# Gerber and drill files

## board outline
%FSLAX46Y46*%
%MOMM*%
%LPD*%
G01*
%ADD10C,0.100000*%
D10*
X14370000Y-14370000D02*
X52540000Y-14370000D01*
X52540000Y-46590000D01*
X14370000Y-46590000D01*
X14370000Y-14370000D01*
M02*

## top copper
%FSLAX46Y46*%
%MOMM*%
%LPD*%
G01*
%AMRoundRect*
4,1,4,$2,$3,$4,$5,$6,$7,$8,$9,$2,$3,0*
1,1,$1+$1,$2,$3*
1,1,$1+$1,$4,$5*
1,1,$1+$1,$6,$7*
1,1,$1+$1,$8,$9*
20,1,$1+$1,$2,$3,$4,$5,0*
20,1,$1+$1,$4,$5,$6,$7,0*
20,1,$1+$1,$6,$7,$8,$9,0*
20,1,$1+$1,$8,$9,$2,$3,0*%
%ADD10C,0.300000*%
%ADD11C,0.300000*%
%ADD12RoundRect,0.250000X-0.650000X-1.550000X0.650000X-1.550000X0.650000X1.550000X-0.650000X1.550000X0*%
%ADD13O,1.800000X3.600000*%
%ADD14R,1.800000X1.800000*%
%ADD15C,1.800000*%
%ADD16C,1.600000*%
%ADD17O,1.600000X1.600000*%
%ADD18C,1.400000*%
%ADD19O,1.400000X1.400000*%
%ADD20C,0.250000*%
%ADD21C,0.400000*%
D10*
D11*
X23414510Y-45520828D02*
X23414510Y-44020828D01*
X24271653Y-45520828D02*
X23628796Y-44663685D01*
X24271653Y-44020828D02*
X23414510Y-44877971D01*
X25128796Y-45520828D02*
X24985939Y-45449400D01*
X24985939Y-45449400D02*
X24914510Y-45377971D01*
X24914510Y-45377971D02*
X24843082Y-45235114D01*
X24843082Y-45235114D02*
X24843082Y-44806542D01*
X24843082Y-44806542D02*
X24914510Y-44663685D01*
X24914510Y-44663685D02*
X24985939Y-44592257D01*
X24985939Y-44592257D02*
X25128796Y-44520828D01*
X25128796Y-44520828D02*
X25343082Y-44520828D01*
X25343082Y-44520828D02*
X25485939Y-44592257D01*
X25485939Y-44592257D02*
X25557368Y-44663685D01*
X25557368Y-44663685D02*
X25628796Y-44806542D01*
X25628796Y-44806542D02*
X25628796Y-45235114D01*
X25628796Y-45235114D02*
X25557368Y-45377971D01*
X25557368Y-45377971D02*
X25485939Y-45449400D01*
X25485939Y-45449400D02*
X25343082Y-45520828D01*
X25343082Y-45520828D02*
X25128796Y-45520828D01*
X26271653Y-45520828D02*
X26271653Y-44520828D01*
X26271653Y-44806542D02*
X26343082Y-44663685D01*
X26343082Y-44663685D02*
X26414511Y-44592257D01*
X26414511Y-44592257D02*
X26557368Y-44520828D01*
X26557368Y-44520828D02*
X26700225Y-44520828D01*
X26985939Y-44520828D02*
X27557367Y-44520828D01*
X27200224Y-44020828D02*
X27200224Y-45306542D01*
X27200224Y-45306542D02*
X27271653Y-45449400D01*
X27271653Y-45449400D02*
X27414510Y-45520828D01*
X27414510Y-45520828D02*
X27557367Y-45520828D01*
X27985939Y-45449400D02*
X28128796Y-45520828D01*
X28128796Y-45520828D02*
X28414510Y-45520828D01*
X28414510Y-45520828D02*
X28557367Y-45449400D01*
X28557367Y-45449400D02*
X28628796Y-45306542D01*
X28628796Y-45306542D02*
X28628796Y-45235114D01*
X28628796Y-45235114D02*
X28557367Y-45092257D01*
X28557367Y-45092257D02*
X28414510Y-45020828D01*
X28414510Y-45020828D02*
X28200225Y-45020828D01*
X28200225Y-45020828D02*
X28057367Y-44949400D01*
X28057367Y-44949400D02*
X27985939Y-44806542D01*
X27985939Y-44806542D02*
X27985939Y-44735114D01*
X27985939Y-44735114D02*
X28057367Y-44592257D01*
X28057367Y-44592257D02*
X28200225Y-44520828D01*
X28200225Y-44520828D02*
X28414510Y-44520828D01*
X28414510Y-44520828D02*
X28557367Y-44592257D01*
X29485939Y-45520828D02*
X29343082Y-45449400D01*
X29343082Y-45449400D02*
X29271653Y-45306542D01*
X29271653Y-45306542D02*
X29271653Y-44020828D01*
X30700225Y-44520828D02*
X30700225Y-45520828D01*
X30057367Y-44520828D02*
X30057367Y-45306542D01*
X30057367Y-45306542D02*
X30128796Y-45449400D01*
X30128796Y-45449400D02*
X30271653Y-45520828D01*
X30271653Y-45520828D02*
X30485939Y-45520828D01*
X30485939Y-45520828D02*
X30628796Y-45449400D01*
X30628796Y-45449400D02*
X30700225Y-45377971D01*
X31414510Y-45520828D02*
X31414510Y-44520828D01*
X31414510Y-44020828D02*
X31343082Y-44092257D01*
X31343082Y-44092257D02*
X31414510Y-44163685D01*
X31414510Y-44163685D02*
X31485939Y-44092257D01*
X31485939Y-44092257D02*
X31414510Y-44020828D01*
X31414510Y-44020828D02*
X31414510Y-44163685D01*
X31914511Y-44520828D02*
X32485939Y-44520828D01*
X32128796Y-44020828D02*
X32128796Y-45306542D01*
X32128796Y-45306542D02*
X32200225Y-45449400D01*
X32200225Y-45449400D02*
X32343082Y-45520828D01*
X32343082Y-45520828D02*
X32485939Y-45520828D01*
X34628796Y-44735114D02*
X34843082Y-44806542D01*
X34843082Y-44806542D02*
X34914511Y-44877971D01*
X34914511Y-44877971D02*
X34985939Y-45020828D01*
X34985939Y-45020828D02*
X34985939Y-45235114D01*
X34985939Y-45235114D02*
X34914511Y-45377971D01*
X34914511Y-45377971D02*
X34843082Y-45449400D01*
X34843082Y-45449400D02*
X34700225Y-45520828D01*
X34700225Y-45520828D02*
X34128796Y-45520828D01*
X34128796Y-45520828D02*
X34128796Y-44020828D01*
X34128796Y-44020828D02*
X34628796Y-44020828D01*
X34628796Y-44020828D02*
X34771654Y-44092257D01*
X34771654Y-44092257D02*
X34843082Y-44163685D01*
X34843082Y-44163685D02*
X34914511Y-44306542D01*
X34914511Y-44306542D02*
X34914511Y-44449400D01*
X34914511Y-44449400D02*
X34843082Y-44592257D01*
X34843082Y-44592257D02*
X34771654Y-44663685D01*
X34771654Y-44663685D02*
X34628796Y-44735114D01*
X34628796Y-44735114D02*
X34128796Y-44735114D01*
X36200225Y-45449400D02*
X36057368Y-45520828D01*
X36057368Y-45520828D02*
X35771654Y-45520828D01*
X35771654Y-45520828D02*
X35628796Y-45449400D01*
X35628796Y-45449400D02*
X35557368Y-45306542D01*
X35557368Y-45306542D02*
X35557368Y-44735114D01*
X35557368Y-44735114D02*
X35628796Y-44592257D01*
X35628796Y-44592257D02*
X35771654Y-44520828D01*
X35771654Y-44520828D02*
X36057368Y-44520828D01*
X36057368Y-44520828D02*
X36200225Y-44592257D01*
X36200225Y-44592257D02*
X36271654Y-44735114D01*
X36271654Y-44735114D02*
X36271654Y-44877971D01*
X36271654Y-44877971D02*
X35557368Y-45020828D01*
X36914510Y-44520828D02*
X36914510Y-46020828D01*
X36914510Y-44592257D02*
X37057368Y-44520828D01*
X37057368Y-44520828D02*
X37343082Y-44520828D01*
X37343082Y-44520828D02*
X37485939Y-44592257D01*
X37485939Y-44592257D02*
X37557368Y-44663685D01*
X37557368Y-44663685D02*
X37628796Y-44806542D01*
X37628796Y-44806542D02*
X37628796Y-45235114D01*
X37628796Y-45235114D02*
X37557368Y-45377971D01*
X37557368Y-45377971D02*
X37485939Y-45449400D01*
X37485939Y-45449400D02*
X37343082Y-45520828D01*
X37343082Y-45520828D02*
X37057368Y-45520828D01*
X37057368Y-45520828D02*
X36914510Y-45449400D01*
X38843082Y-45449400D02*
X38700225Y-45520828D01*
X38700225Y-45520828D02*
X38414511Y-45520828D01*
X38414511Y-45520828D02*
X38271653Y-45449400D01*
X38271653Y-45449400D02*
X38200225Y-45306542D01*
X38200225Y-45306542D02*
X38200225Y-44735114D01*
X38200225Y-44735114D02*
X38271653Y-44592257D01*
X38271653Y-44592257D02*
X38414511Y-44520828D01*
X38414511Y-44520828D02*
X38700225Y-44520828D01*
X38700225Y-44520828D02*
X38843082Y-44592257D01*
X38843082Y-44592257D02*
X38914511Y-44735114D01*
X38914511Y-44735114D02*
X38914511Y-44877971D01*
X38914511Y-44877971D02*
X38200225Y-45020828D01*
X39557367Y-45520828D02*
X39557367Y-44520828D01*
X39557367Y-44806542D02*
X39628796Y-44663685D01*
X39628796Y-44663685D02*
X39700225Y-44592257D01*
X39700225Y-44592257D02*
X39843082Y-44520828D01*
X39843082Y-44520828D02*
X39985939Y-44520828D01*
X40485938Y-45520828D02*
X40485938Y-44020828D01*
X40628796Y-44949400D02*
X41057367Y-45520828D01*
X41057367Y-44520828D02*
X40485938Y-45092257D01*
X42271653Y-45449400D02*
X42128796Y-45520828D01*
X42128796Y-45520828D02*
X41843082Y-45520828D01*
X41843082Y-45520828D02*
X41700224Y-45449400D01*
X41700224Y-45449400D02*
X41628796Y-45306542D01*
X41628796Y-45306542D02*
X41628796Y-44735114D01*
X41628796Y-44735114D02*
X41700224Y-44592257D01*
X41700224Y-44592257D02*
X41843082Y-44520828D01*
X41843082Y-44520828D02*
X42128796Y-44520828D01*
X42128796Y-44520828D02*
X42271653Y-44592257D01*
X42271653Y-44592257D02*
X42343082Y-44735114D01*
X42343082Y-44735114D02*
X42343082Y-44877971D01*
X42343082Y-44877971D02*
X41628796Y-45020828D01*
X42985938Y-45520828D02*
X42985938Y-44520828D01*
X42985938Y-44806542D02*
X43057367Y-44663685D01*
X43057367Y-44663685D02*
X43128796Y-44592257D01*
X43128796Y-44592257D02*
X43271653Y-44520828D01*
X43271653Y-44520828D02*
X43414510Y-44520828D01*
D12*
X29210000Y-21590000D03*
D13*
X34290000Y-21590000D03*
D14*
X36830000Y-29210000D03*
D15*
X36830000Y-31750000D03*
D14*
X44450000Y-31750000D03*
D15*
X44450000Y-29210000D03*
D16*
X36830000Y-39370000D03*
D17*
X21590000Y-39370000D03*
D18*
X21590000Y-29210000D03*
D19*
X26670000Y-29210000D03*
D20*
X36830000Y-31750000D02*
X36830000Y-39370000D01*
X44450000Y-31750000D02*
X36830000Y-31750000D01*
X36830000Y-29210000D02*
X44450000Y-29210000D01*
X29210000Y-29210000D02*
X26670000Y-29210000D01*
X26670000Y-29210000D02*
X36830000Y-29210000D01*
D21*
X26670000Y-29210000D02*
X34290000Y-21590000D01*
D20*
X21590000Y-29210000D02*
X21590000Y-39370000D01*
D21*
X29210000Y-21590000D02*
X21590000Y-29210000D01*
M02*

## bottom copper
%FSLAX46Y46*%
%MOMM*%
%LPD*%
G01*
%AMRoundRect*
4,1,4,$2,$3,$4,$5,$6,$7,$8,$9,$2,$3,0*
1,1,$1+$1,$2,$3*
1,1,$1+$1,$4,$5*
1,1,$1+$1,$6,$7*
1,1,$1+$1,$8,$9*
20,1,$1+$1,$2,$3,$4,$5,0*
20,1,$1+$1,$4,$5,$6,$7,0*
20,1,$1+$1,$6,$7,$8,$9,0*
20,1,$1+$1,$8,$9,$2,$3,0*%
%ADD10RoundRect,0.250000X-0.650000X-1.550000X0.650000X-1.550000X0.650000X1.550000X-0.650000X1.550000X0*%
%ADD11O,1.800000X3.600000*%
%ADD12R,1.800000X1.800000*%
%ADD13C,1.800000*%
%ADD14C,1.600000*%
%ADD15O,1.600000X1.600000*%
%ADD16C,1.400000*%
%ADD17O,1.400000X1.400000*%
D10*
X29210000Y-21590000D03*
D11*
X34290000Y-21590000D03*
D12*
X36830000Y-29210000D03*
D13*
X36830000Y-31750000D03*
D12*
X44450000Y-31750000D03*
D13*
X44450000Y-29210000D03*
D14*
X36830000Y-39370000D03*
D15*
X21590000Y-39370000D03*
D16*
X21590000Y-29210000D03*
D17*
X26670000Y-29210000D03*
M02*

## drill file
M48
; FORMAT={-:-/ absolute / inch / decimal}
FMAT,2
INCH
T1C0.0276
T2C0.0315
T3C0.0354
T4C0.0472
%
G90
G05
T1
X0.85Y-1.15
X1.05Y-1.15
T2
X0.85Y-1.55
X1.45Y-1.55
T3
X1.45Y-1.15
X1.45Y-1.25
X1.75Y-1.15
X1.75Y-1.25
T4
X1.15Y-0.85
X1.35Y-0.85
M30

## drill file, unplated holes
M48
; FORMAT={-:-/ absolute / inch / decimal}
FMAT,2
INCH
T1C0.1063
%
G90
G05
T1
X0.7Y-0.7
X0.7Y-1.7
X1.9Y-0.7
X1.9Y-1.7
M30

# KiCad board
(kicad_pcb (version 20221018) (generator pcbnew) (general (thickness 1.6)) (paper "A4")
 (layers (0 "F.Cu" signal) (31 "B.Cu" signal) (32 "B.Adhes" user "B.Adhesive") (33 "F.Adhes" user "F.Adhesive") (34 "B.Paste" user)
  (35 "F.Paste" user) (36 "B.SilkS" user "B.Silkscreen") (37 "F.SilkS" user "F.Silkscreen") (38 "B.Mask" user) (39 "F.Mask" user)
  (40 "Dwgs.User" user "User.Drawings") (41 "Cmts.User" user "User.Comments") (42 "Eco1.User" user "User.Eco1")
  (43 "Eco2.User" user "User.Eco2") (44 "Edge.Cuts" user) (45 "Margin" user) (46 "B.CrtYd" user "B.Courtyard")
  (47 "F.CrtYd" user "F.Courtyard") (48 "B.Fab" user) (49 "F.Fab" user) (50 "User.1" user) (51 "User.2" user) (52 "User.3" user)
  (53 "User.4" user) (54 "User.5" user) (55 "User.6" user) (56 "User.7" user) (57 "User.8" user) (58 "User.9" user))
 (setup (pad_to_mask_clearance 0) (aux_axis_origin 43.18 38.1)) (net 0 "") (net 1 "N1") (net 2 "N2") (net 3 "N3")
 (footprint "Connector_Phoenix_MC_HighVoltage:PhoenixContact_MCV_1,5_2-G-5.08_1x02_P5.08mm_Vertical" (layer "F.Cu") (at 29.21 21.59)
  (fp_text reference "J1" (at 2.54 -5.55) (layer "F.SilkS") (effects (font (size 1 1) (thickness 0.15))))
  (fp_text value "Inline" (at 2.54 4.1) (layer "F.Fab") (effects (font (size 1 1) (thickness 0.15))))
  (pad "1" thru_hole roundrect (at 0 0) (size 1.8 3.6) (drill 1.2) (layers "*.Cu" "*.Mask") (roundrect_rratio 0.1388888889) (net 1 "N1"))
  (pad "2" thru_hole oval (at 5.08 0) (size 1.8 3.6) (drill 1.2) (layers "*.Cu" "*.Mask") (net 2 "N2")))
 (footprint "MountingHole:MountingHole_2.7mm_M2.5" (layer "F.Cu") (at 17.78 17.78)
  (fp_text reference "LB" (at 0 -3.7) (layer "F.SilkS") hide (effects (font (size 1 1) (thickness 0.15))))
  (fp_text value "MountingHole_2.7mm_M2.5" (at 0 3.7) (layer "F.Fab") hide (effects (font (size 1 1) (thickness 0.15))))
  (pad "" np_thru_hole circle (at 0 0) (size 2.7 2.7) (drill 2.7) (layers "*.Cu" "*.Mask")))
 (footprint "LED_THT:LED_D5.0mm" (layer "F.Cu") (at 36.83 29.21 -90)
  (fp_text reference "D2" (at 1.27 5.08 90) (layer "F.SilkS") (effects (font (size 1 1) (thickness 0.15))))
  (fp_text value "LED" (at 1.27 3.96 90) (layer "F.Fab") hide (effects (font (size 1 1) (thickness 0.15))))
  (pad "1" thru_hole rect (at 0 0 270) (size 1.8 1.8) (drill 0.9) (layers "*.Cu" "*.Mask") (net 2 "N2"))
  (pad "2" thru_hole circle (at 2.54 0 270) (size 1.8 1.8) (drill 0.9) (layers "*.Cu" "*.Mask") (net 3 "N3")))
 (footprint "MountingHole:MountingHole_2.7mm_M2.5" (layer "F.Cu") (at 17.78 43.18)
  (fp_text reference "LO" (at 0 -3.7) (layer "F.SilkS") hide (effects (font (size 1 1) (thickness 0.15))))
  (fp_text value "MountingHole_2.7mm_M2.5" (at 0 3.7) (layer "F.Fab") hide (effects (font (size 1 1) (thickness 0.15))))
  (pad "" np_thru_hole circle (at 0 0) (size 2.7 2.7) (drill 2.7) (layers "*.Cu" "*.Mask")))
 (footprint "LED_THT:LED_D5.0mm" (layer "F.Cu") (at 44.45 31.75 90)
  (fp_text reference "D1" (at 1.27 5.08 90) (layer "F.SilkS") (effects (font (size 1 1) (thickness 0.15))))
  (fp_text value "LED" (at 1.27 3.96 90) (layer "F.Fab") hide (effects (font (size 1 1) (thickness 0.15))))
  (pad "1" thru_hole rect (at 0 0 90) (size 1.8 1.8) (drill 0.9) (layers "*.Cu" "*.Mask") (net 3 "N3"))
  (pad "2" thru_hole circle (at 2.54 0 90) (size 1.8 1.8) (drill 0.9) (layers "*.Cu" "*.Mask") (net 2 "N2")))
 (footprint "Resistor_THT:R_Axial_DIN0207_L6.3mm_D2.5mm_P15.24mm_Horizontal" (layer "F.Cu") (at 36.83 39.37 180)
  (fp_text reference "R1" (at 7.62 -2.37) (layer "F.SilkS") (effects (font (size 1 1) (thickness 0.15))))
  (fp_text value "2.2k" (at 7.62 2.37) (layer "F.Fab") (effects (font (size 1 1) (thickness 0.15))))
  (pad "1" thru_hole circle (at 0 0 180) (size 1.6 1.6) (drill 0.8) (layers "*.Cu" "*.Mask") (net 3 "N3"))
  (pad "2" thru_hole oval (at 15.24 0 180) (size 1.6 1.6) (drill 0.8) (layers "*.Cu" "*.Mask") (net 1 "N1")))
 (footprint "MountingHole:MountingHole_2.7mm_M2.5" (layer "F.Cu") (at 48.26 43.18)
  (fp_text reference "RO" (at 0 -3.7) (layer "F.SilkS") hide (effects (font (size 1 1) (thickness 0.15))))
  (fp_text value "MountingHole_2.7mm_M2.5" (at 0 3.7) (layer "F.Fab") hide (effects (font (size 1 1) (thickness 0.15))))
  (pad "" np_thru_hole circle (at 0 0) (size 2.7 2.7) (drill 2.7) (layers "*.Cu" "*.Mask")))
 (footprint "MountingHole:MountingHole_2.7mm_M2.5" (layer "F.Cu") (at 48.26 17.78)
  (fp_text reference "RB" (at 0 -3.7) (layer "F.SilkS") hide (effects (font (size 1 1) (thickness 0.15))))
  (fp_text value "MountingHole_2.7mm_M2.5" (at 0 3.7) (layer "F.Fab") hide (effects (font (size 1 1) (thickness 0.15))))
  (pad "" np_thru_hole circle (at 0 0) (size 2.7 2.7) (drill 2.7) (layers "*.Cu" "*.Mask")))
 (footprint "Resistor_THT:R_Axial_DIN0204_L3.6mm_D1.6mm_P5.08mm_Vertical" (layer "F.Cu") (at 21.59 29.21)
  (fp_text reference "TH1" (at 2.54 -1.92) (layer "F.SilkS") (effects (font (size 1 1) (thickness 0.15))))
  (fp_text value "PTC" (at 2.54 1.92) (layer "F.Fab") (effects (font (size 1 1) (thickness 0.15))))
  (pad "1" thru_hole circle (at 0 0) (size 1.4 1.4) (drill 0.7) (layers "*.Cu" "*.Mask") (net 1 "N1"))
  (pad "2" thru_hole oval (at 5.08 0) (size 1.4 1.4) (drill 0.7) (layers "*.Cu" "*.Mask") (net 2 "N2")))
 (gr_rect (start 14.37 14.37) (end 52.54 46.59) (stroke (width 0.1) (type default)) (fill none) (layer "Edge.Cuts"))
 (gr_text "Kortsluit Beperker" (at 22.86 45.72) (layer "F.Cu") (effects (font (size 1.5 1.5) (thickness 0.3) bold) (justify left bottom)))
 (segment (start 36.83 31.75) (end 36.83 39.37) (width 0.25) (layer "F.Cu") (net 3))
 (segment (start 44.45 31.75) (end 36.83 31.75) (width 0.25) (layer "F.Cu") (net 3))
 (segment (start 36.83 29.21) (end 44.45 29.21) (width 0.25) (layer "F.Cu") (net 2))
 (segment (start 29.21 29.21) (end 26.67 29.21) (width 0.25) (layer "F.Cu") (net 2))
 (segment (start 26.67 29.21) (end 36.83 29.21) (width 0.25) (layer "F.Cu") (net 2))
 (segment (start 26.67 29.21) (end 34.29 21.59) (width 0.4) (layer "F.Cu") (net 2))
 (segment (start 21.59 29.21) (end 21.59 39.37) (width 0.25) (layer "F.Cu") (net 1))
 (segment (start 29.21 21.59) (end 21.59 29.21) (width 0.4) (layer "F.Cu") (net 1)))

